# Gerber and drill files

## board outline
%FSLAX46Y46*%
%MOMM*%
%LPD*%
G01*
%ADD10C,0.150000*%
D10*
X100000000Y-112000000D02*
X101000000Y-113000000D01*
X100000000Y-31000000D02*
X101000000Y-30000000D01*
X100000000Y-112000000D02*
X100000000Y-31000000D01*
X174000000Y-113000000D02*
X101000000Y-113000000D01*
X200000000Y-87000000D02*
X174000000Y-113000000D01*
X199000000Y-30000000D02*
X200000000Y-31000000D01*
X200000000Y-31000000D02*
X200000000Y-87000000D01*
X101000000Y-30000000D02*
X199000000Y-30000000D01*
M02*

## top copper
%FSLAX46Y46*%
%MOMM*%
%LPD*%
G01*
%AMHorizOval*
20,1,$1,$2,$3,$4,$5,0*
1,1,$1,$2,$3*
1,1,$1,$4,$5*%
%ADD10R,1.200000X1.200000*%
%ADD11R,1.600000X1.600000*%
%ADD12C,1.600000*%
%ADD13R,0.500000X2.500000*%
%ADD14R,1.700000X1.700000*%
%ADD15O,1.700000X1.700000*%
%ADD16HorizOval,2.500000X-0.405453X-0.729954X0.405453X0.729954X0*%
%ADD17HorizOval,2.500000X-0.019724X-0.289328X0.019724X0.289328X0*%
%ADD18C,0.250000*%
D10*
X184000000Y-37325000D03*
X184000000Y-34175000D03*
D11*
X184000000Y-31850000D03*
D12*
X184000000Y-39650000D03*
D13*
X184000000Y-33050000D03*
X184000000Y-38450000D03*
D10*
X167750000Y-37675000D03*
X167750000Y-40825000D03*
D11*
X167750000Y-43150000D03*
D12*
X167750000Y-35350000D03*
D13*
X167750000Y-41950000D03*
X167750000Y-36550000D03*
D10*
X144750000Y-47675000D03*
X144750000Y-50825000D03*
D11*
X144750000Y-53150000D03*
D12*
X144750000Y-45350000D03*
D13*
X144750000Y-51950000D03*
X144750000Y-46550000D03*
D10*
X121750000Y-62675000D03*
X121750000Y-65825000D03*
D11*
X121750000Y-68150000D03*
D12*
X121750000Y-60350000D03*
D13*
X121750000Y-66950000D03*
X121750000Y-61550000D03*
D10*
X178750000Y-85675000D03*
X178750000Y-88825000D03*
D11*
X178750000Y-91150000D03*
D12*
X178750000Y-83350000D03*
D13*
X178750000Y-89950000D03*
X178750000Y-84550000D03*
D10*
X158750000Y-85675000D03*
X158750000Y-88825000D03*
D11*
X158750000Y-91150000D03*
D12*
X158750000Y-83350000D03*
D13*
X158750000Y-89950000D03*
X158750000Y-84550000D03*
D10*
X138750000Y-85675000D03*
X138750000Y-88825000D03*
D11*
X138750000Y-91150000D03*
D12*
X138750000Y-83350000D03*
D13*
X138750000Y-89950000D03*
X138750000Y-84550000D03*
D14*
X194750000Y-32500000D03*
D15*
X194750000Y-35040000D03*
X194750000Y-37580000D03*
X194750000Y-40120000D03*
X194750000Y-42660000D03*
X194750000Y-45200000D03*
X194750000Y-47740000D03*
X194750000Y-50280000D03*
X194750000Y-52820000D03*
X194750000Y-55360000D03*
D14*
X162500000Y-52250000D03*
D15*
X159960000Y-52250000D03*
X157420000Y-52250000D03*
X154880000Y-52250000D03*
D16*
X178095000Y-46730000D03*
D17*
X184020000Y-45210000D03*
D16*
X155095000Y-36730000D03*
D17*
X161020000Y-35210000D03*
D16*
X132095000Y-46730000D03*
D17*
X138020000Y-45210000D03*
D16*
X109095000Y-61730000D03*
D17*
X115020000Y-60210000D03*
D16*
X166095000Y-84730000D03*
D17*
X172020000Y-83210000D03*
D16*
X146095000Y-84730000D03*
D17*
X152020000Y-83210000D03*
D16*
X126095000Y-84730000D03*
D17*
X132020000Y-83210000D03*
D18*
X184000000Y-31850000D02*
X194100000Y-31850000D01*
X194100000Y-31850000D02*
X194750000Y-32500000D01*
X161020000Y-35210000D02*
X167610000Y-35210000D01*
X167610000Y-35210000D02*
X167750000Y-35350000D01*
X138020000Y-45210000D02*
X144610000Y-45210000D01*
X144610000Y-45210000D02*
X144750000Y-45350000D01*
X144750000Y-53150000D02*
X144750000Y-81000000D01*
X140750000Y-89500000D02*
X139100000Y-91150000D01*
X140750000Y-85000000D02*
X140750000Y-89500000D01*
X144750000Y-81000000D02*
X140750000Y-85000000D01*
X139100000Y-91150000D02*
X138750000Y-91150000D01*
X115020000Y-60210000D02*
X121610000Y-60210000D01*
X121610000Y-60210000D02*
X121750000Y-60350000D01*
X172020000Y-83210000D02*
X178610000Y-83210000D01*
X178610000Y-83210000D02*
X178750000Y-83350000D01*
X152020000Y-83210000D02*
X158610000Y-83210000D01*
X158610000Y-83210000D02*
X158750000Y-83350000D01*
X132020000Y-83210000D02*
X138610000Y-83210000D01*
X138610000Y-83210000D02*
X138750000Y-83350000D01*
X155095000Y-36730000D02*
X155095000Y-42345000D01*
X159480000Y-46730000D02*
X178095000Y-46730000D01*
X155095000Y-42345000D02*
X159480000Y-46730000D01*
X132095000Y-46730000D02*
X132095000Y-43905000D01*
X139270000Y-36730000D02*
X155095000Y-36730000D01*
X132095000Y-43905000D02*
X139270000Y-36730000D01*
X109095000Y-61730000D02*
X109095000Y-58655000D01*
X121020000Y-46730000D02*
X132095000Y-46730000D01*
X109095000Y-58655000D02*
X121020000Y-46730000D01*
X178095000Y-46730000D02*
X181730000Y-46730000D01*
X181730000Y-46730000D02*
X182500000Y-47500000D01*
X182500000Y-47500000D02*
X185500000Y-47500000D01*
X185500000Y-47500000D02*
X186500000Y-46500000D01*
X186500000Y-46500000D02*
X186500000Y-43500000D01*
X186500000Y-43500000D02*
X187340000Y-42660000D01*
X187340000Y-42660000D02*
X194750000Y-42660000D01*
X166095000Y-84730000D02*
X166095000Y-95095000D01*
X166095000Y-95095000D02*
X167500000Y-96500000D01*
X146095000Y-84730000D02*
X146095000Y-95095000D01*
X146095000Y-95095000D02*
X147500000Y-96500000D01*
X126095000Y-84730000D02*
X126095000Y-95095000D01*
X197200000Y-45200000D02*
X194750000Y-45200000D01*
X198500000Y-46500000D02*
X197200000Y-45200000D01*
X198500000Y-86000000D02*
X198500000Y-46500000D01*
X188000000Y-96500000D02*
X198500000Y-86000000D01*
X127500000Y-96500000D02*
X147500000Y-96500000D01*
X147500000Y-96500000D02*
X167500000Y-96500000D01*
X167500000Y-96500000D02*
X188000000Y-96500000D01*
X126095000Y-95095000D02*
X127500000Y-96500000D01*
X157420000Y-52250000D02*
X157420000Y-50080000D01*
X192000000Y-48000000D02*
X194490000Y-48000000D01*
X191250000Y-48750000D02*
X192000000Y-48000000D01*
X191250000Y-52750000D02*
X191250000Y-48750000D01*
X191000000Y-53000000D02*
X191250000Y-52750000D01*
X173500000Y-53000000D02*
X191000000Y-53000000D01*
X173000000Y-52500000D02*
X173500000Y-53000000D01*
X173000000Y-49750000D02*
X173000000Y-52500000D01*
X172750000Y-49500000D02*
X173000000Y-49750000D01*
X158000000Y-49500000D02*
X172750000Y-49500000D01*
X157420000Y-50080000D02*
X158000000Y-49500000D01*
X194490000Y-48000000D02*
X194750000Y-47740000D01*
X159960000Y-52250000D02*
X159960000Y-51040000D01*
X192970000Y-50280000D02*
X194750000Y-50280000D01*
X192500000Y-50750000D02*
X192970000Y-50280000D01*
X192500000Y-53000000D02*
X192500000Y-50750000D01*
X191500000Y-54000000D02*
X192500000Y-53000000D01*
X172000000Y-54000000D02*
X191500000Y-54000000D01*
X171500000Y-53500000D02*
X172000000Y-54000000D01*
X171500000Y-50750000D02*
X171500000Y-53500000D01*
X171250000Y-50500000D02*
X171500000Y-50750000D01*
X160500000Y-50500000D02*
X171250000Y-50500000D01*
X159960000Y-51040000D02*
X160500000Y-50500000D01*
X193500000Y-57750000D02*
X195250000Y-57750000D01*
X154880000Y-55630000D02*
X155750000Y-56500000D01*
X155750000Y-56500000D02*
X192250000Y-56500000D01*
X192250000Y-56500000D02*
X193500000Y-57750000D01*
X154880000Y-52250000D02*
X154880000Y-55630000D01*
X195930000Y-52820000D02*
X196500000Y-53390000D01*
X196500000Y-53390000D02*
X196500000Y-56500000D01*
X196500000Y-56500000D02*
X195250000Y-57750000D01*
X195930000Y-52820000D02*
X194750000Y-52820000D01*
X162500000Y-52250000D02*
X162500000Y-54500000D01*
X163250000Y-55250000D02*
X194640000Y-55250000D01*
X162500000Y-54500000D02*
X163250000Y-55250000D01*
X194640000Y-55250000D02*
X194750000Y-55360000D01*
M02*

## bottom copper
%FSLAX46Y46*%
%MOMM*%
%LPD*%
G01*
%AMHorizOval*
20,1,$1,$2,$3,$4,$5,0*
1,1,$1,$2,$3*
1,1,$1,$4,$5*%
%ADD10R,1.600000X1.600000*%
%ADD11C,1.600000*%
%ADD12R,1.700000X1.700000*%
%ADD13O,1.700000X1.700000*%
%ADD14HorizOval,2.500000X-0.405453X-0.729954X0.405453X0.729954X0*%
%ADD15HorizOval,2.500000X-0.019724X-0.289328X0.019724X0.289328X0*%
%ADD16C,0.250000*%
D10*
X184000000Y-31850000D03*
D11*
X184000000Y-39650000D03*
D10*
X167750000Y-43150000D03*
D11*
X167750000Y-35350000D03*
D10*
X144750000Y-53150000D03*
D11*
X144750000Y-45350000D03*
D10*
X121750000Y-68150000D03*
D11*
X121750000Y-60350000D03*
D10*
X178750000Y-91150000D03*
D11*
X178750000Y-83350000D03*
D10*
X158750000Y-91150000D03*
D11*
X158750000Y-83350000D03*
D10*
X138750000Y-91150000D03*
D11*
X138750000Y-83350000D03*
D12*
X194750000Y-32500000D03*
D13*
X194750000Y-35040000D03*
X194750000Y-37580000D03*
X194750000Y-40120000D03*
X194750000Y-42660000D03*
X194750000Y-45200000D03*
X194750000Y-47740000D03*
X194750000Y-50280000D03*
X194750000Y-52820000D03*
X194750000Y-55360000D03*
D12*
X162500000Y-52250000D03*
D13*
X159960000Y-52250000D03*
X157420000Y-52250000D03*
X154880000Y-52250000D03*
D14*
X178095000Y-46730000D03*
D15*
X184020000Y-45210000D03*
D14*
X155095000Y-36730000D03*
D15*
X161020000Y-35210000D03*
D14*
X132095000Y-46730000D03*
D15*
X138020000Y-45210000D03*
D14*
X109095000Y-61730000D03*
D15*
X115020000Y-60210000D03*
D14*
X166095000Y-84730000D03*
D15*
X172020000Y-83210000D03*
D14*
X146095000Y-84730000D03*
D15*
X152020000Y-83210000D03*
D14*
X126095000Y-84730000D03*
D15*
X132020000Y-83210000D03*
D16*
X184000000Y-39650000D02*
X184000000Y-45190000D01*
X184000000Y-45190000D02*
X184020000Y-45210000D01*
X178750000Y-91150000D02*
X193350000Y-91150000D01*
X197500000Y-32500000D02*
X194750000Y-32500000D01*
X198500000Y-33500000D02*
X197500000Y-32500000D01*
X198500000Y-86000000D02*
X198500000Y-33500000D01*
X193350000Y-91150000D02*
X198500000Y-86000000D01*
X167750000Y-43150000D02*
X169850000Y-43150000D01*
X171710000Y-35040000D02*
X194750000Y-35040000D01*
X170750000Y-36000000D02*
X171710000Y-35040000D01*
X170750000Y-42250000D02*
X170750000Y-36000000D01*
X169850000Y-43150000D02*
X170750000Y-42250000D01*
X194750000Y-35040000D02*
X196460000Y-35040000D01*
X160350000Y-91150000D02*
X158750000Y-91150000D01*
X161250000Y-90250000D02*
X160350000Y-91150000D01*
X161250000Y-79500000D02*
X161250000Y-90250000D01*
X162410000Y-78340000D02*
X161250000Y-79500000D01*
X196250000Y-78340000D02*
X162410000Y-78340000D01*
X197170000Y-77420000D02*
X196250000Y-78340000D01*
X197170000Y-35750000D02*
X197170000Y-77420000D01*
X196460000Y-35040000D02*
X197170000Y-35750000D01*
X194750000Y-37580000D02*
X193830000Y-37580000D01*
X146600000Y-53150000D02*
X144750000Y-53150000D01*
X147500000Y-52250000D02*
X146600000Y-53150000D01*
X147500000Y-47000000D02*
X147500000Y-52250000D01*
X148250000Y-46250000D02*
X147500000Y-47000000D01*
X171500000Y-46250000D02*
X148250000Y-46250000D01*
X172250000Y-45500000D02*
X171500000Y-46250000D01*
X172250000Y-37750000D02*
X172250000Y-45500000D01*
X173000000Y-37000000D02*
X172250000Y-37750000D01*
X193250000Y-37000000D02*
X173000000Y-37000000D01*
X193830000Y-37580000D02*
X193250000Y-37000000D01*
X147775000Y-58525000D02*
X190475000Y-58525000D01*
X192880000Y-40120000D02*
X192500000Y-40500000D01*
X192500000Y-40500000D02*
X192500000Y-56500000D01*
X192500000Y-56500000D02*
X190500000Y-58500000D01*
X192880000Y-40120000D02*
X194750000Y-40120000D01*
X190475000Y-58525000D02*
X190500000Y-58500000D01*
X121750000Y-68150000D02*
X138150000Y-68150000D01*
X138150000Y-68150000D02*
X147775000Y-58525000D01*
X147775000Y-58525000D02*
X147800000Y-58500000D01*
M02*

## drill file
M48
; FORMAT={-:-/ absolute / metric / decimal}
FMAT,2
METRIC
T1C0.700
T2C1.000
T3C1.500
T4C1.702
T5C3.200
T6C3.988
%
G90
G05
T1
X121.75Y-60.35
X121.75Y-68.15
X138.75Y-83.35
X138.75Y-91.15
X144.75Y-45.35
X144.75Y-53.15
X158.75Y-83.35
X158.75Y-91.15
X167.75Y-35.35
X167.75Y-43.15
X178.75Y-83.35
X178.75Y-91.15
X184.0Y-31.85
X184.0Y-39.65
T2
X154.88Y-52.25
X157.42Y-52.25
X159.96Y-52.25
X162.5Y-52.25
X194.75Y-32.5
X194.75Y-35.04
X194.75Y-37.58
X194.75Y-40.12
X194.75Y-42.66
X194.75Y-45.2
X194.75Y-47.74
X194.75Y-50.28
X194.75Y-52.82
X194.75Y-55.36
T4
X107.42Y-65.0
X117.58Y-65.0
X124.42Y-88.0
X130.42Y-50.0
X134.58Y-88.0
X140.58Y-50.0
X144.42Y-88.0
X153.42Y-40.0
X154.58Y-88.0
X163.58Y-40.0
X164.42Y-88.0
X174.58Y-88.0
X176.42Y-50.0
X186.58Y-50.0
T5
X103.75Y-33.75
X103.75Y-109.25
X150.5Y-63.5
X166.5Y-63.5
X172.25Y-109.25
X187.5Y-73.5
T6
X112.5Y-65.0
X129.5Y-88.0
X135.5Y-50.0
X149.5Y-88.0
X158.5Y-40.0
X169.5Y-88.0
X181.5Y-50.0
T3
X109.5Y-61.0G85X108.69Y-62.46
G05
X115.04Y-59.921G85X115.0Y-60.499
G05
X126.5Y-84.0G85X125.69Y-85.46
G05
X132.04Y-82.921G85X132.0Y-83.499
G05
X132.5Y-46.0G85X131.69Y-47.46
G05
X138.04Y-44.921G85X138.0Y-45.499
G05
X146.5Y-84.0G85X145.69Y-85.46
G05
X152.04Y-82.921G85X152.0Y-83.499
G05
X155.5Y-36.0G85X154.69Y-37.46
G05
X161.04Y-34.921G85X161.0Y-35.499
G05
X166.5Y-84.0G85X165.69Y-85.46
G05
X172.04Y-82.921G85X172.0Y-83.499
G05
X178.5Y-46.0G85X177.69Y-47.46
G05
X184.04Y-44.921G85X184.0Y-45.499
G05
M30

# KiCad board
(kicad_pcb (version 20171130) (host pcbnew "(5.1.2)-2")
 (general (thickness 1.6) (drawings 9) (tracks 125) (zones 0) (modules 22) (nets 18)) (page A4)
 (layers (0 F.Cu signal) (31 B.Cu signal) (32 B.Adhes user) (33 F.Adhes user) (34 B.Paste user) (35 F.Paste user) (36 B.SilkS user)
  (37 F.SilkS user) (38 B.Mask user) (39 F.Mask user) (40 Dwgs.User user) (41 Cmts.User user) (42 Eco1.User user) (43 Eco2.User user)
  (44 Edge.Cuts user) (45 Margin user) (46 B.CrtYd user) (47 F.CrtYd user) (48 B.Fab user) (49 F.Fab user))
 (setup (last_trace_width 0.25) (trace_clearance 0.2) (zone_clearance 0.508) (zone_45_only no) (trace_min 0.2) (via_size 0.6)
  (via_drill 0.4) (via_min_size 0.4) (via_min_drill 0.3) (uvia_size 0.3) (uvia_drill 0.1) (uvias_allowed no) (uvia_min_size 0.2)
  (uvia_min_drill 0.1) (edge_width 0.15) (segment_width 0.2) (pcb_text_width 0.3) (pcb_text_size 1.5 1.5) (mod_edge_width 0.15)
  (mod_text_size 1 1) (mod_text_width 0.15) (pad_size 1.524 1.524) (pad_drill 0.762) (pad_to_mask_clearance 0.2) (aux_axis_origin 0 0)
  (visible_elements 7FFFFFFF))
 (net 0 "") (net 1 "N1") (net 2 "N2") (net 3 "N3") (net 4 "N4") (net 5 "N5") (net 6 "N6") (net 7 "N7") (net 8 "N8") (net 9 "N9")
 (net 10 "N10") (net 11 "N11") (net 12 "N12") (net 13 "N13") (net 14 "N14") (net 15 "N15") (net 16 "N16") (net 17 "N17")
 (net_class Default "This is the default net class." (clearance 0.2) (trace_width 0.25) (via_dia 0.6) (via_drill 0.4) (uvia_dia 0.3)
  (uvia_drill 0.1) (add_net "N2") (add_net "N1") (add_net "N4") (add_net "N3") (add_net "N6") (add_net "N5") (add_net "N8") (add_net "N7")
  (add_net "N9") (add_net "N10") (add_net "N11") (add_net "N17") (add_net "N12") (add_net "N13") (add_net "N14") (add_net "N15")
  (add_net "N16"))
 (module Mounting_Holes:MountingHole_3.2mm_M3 (layer F.Cu) (at 187.5 73.5)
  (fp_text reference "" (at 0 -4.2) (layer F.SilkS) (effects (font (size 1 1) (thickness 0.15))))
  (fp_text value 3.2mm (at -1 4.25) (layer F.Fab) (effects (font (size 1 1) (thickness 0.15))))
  (pad 1 np_thru_hole circle (at 0 0) (size 3.2 3.2) (drill 3.2) (layers *.Cu *.Mask)))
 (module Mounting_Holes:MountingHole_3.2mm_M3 (layer F.Cu) (at 172.25 109.25)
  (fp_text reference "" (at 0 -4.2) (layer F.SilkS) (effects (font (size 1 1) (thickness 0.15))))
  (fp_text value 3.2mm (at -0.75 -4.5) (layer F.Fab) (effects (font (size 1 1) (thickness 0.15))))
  (pad 1 np_thru_hole circle (at 0 0) (size 3.2 3.2) (drill 3.2) (layers *.Cu *.Mask)))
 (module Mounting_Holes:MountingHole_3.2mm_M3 (layer F.Cu) (at 103.75 109.25)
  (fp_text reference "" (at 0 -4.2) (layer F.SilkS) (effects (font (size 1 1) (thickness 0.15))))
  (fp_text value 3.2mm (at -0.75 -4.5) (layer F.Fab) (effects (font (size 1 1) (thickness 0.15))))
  (pad 1 np_thru_hole circle (at 0 0) (size 3.2 3.2) (drill 3.2) (layers *.Cu *.Mask)))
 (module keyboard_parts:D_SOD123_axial (layer F.Cu) (at 184 35.75 270)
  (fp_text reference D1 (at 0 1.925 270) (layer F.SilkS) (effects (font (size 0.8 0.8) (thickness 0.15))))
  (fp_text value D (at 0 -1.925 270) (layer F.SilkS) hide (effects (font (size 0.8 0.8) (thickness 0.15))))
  (pad 2 smd rect (at 1.575 0 270) (size 1.2 1.2) (layers F.Cu F.Paste F.Mask) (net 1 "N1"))
  (pad 1 smd rect (at -1.575 0 270) (size 1.2 1.2) (layers F.Cu F.Paste F.Mask) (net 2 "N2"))
  (pad 1 thru_hole rect (at -3.9 0 270) (size 1.6 1.6) (drill 0.7) (layers *.Cu *.Mask F.SilkS) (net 2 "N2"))
  (pad 2 thru_hole circle (at 3.9 0 270) (size 1.6 1.6) (drill 0.7) (layers *.Cu *.Mask F.SilkS) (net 1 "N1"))
  (pad 1 smd rect (at -2.7 0 270) (size 2.5 0.5) (layers F.Cu) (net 2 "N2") (solder_mask_margin -999))
  (pad 2 smd rect (at 2.7 0 270) (size 2.5 0.5) (layers F.Cu) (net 1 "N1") (solder_mask_margin -999)))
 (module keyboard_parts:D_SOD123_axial (layer F.Cu) (at 167.75 39.25 90)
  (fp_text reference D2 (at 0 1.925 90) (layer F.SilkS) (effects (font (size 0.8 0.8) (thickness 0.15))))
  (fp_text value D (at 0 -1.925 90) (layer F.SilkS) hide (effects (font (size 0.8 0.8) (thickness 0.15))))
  (pad 2 smd rect (at 1.575 0 90) (size 1.2 1.2) (layers F.Cu F.Paste F.Mask) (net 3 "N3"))
  (pad 1 smd rect (at -1.575 0 90) (size 1.2 1.2) (layers F.Cu F.Paste F.Mask) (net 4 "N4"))
  (pad 1 thru_hole rect (at -3.9 0 90) (size 1.6 1.6) (drill 0.7) (layers *.Cu *.Mask F.SilkS) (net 4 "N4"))
  (pad 2 thru_hole circle (at 3.9 0 90) (size 1.6 1.6) (drill 0.7) (layers *.Cu *.Mask F.SilkS) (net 3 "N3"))
  (pad 1 smd rect (at -2.7 0 90) (size 2.5 0.5) (layers F.Cu) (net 4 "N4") (solder_mask_margin -999))
  (pad 2 smd rect (at 2.7 0 90) (size 2.5 0.5) (layers F.Cu) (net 3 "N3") (solder_mask_margin -999)))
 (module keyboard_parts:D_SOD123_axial (layer F.Cu) (at 144.75 49.25 90)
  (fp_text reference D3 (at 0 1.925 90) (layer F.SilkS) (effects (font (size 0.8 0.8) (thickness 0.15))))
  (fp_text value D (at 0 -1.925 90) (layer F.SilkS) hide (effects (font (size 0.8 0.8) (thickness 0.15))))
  (pad 2 smd rect (at 1.575 0 90) (size 1.2 1.2) (layers F.Cu F.Paste F.Mask) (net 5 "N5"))
  (pad 1 smd rect (at -1.575 0 90) (size 1.2 1.2) (layers F.Cu F.Paste F.Mask) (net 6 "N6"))
  (pad 1 thru_hole rect (at -3.9 0 90) (size 1.6 1.6) (drill 0.7) (layers *.Cu *.Mask F.SilkS) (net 6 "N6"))
  (pad 2 thru_hole circle (at 3.9 0 90) (size 1.6 1.6) (drill 0.7) (layers *.Cu *.Mask F.SilkS) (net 5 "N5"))
  (pad 1 smd rect (at -2.7 0 90) (size 2.5 0.5) (layers F.Cu) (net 6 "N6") (solder_mask_margin -999))
  (pad 2 smd rect (at 2.7 0 90) (size 2.5 0.5) (layers F.Cu) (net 5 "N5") (solder_mask_margin -999)))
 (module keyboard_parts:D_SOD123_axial (layer F.Cu) (at 121.75 64.25 90)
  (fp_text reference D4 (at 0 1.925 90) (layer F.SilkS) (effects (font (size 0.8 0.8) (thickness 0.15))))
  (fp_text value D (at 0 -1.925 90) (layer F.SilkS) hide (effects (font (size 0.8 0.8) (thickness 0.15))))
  (pad 2 smd rect (at 1.575 0 90) (size 1.2 1.2) (layers F.Cu F.Paste F.Mask) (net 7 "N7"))
  (pad 1 smd rect (at -1.575 0 90) (size 1.2 1.2) (layers F.Cu F.Paste F.Mask) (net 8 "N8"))
  (pad 1 thru_hole rect (at -3.9 0 90) (size 1.6 1.6) (drill 0.7) (layers *.Cu *.Mask F.SilkS) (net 8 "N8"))
  (pad 2 thru_hole circle (at 3.9 0 90) (size 1.6 1.6) (drill 0.7) (layers *.Cu *.Mask F.SilkS) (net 7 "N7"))
  (pad 1 smd rect (at -2.7 0 90) (size 2.5 0.5) (layers F.Cu) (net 8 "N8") (solder_mask_margin -999))
  (pad 2 smd rect (at 2.7 0 90) (size 2.5 0.5) (layers F.Cu) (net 7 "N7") (solder_mask_margin -999)))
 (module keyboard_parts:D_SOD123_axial (layer F.Cu) (at 178.75 87.25 90)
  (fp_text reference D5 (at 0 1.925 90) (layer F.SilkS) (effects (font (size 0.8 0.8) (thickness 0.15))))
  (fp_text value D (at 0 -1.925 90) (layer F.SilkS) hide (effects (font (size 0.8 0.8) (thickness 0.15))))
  (pad 2 smd rect (at 1.575 0 90) (size 1.2 1.2) (layers F.Cu F.Paste F.Mask) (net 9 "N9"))
  (pad 1 smd rect (at -1.575 0 90) (size 1.2 1.2) (layers F.Cu F.Paste F.Mask) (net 2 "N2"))
  (pad 1 thru_hole rect (at -3.9 0 90) (size 1.6 1.6) (drill 0.7) (layers *.Cu *.Mask F.SilkS) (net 2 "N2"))
  (pad 2 thru_hole circle (at 3.9 0 90) (size 1.6 1.6) (drill 0.7) (layers *.Cu *.Mask F.SilkS) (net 9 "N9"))
  (pad 1 smd rect (at -2.7 0 90) (size 2.5 0.5) (layers F.Cu) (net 2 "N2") (solder_mask_margin -999))
  (pad 2 smd rect (at 2.7 0 90) (size 2.5 0.5) (layers F.Cu) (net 9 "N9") (solder_mask_margin -999)))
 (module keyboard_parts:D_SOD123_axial (layer F.Cu) (at 158.75 87.25 90)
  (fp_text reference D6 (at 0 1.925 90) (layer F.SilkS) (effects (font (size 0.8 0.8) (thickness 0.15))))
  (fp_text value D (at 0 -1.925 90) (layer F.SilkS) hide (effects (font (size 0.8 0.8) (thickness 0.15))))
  (pad 2 smd rect (at 1.575 0 90) (size 1.2 1.2) (layers F.Cu F.Paste F.Mask) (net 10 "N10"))
  (pad 1 smd rect (at -1.575 0 90) (size 1.2 1.2) (layers F.Cu F.Paste F.Mask) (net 4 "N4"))
  (pad 1 thru_hole rect (at -3.9 0 90) (size 1.6 1.6) (drill 0.7) (layers *.Cu *.Mask F.SilkS) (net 4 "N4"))
  (pad 2 thru_hole circle (at 3.9 0 90) (size 1.6 1.6) (drill 0.7) (layers *.Cu *.Mask F.SilkS) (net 10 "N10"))
  (pad 1 smd rect (at -2.7 0 90) (size 2.5 0.5) (layers F.Cu) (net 4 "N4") (solder_mask_margin -999))
  (pad 2 smd rect (at 2.7 0 90) (size 2.5 0.5) (layers F.Cu) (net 10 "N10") (solder_mask_margin -999)))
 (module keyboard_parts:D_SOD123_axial (layer F.Cu) (at 138.75 87.25 90)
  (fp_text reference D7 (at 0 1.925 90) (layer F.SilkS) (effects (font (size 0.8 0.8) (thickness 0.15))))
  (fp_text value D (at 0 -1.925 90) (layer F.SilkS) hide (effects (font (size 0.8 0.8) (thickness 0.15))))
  (pad 2 smd rect (at 1.575 0 90) (size 1.2 1.2) (layers F.Cu F.Paste F.Mask) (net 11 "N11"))
  (pad 1 smd rect (at -1.575 0 90) (size 1.2 1.2) (layers F.Cu F.Paste F.Mask) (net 6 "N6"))
  (pad 1 thru_hole rect (at -3.9 0 90) (size 1.6 1.6) (drill 0.7) (layers *.Cu *.Mask F.SilkS) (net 6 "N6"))
  (pad 2 thru_hole circle (at 3.9 0 90) (size 1.6 1.6) (drill 0.7) (layers *.Cu *.Mask F.SilkS) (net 11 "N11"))
  (pad 1 smd rect (at -2.7 0 90) (size 2.5 0.5) (layers F.Cu) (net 6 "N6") (solder_mask_margin -999))
  (pad 2 smd rect (at 2.7 0 90) (size 2.5 0.5) (layers F.Cu) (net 11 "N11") (solder_mask_margin -999)))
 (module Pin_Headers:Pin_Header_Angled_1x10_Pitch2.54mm (layer F.Cu) (at 194.75 32.5)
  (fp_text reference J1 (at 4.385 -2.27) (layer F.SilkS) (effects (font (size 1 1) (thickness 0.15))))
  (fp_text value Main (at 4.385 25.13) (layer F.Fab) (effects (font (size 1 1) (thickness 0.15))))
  (pad 1 thru_hole rect (at 0 0) (size 1.7 1.7) (drill 1) (layers *.Cu *.Mask) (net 2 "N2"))
  (pad 2 thru_hole oval (at 0 2.54) (size 1.7 1.7) (drill 1) (layers *.Cu *.Mask) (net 4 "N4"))
  (pad 3 thru_hole oval (at 0 5.08) (size 1.7 1.7) (drill 1) (layers *.Cu *.Mask) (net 6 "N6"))
  (pad 4 thru_hole oval (at 0 7.62) (size 1.7 1.7) (drill 1) (layers *.Cu *.Mask) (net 8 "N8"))
  (pad 5 thru_hole oval (at 0 10.16) (size 1.7 1.7) (drill 1) (layers *.Cu *.Mask) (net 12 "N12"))
  (pad 6 thru_hole oval (at 0 12.7) (size 1.7 1.7) (drill 1) (layers *.Cu *.Mask) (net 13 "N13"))
  (pad 7 thru_hole oval (at 0 15.24) (size 1.7 1.7) (drill 1) (layers *.Cu *.Mask) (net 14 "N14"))
  (pad 8 thru_hole oval (at 0 17.78) (size 1.7 1.7) (drill 1) (layers *.Cu *.Mask) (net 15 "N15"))
  (pad 9 thru_hole oval (at 0 20.32) (size 1.7 1.7) (drill 1) (layers *.Cu *.Mask) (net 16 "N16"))
  (pad 10 thru_hole oval (at 0 22.86) (size 1.7 1.7) (drill 1) (layers *.Cu *.Mask) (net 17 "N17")))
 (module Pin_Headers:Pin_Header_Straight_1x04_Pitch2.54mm (layer F.Cu) (at 162.5 52.25 270)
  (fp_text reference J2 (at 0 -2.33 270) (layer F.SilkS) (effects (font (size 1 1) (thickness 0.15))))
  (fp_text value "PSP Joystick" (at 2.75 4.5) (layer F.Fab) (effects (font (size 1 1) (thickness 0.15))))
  (pad 1 thru_hole rect (at 0 0 270) (size 1.7 1.7) (drill 1) (layers *.Cu *.Mask) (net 17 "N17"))
  (pad 2 thru_hole oval (at 0 2.54 270) (size 1.7 1.7) (drill 1) (layers *.Cu *.Mask) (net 15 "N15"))
  (pad 3 thru_hole oval (at 0 5.08 270) (size 1.7 1.7) (drill 1) (layers *.Cu *.Mask) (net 14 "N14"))
  (pad 4 thru_hole oval (at 0 7.62 270) (size 1.7 1.7) (drill 1) (layers *.Cu *.Mask) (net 16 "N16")))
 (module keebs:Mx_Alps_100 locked (layer F.Cu) (at 181.5 50)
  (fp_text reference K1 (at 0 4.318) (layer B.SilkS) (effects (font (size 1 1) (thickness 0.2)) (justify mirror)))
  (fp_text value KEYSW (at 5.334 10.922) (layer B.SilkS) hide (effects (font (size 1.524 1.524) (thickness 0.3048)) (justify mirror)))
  (pad HOLE np_thru_hole circle (at 0 0) (size 3.9878 3.9878) (drill 3.9878) (layers *.Cu))
  (pad HOLE np_thru_hole circle (at -5.08 0) (size 1.7018 1.7018) (drill 1.7018) (layers *.Cu))
  (pad HOLE np_thru_hole circle (at 5.08 0) (size 1.7018 1.7018) (drill 1.7018) (layers *.Cu))
  (pad 1 thru_hole oval (at -3.405 -3.27 330.95) (size 2.5 4.17) (drill oval 1.5 3.17) (layers *.Cu *.Mask F.SilkS) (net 12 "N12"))
  (pad 2 thru_hole oval (at 2.52 -4.79 356.1) (size 2.5 3.08) (drill oval 1.5 2.08) (layers *.Cu *.Mask F.SilkS) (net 1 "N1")))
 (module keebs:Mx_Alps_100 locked (layer F.Cu) (at 158.5 40)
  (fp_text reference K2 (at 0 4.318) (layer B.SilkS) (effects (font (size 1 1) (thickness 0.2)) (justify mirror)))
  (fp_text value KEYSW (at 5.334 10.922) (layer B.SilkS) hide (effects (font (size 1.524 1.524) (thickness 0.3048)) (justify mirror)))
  (pad HOLE np_thru_hole circle (at 0 0) (size 3.9878 3.9878) (drill 3.9878) (layers *.Cu))
  (pad HOLE np_thru_hole circle (at -5.08 0) (size 1.7018 1.7018) (drill 1.7018) (layers *.Cu))
  (pad HOLE np_thru_hole circle (at 5.08 0) (size 1.7018 1.7018) (drill 1.7018) (layers *.Cu))
  (pad 1 thru_hole oval (at -3.405 -3.27 330.95) (size 2.5 4.17) (drill oval 1.5 3.17) (layers *.Cu *.Mask F.SilkS) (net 12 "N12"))
  (pad 2 thru_hole oval (at 2.52 -4.79 356.1) (size 2.5 3.08) (drill oval 1.5 2.08) (layers *.Cu *.Mask F.SilkS) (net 3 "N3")))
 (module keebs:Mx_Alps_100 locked (layer F.Cu) (at 135.5 50)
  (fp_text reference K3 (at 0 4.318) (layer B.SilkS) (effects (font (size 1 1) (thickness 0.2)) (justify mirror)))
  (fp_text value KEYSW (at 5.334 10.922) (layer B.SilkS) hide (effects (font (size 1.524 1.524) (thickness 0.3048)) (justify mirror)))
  (pad HOLE np_thru_hole circle (at 0 0) (size 3.9878 3.9878) (drill 3.9878) (layers *.Cu))
  (pad HOLE np_thru_hole circle (at -5.08 0) (size 1.7018 1.7018) (drill 1.7018) (layers *.Cu))
  (pad HOLE np_thru_hole circle (at 5.08 0) (size 1.7018 1.7018) (drill 1.7018) (layers *.Cu))
  (pad 1 thru_hole oval (at -3.405 -3.27 330.95) (size 2.5 4.17) (drill oval 1.5 3.17) (layers *.Cu *.Mask F.SilkS) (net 12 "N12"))
  (pad 2 thru_hole oval (at 2.52 -4.79 356.1) (size 2.5 3.08) (drill oval 1.5 2.08) (layers *.Cu *.Mask F.SilkS) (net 5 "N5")))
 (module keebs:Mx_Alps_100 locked (layer F.Cu) (at 112.5 65)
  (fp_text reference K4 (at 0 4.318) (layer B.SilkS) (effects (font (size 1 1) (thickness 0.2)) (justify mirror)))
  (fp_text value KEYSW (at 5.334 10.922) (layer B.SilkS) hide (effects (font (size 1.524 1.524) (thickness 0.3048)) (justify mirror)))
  (pad HOLE np_thru_hole circle (at 0 0) (size 3.9878 3.9878) (drill 3.9878) (layers *.Cu))
  (pad HOLE np_thru_hole circle (at -5.08 0) (size 1.7018 1.7018) (drill 1.7018) (layers *.Cu))
  (pad HOLE np_thru_hole circle (at 5.08 0) (size 1.7018 1.7018) (drill 1.7018) (layers *.Cu))
  (pad 1 thru_hole oval (at -3.405 -3.27 330.95) (size 2.5 4.17) (drill oval 1.5 3.17) (layers *.Cu *.Mask F.SilkS) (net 12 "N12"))
  (pad 2 thru_hole oval (at 2.52 -4.79 356.1) (size 2.5 3.08) (drill oval 1.5 2.08) (layers *.Cu *.Mask F.SilkS) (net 7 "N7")))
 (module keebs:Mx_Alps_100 (layer F.Cu) (at 169.5 88)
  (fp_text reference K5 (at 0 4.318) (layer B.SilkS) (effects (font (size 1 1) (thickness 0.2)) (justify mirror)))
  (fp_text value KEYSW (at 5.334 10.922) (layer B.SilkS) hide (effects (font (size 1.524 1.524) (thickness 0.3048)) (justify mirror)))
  (pad HOLE np_thru_hole circle (at 0 0) (size 3.9878 3.9878) (drill 3.9878) (layers *.Cu))
  (pad HOLE np_thru_hole circle (at -5.08 0) (size 1.7018 1.7018) (drill 1.7018) (layers *.Cu))
  (pad HOLE np_thru_hole circle (at 5.08 0) (size 1.7018 1.7018) (drill 1.7018) (layers *.Cu))
  (pad 1 thru_hole oval (at -3.405 -3.27 330.95) (size 2.5 4.17) (drill oval 1.5 3.17) (layers *.Cu *.Mask F.SilkS) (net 13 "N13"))
  (pad 2 thru_hole oval (at 2.52 -4.79 356.1) (size 2.5 3.08) (drill oval 1.5 2.08) (layers *.Cu *.Mask F.SilkS) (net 9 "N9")))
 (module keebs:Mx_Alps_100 (layer F.Cu) (at 149.5 88)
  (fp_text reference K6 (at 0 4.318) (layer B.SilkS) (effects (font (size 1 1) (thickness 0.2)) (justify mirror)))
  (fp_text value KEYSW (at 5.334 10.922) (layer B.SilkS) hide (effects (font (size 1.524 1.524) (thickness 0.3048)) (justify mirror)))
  (pad HOLE np_thru_hole circle (at 0 0) (size 3.9878 3.9878) (drill 3.9878) (layers *.Cu))
  (pad HOLE np_thru_hole circle (at -5.08 0) (size 1.7018 1.7018) (drill 1.7018) (layers *.Cu))
  (pad HOLE np_thru_hole circle (at 5.08 0) (size 1.7018 1.7018) (drill 1.7018) (layers *.Cu))
  (pad 1 thru_hole oval (at -3.405 -3.27 330.95) (size 2.5 4.17) (drill oval 1.5 3.17) (layers *.Cu *.Mask F.SilkS) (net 13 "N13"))
  (pad 2 thru_hole oval (at 2.52 -4.79 356.1) (size 2.5 3.08) (drill oval 1.5 2.08) (layers *.Cu *.Mask F.SilkS) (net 10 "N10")))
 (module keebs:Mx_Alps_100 (layer F.Cu) (at 129.5 88)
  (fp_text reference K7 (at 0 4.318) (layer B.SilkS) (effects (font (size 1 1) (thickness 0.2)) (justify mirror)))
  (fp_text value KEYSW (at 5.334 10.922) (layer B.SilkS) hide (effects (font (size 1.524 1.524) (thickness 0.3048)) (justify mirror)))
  (pad HOLE np_thru_hole circle (at 0 0) (size 3.9878 3.9878) (drill 3.9878) (layers *.Cu))
  (pad HOLE np_thru_hole circle (at -5.08 0) (size 1.7018 1.7018) (drill 1.7018) (layers *.Cu))
  (pad HOLE np_thru_hole circle (at 5.08 0) (size 1.7018 1.7018) (drill 1.7018) (layers *.Cu))
  (pad 1 thru_hole oval (at -3.405 -3.27 330.95) (size 2.5 4.17) (drill oval 1.5 3.17) (layers *.Cu *.Mask F.SilkS) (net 13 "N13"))
  (pad 2 thru_hole oval (at 2.52 -4.79 356.1) (size 2.5 3.08) (drill oval 1.5 2.08) (layers *.Cu *.Mask F.SilkS) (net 11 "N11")))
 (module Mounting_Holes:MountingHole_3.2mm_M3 (layer F.Cu) (at 166.5 63.5)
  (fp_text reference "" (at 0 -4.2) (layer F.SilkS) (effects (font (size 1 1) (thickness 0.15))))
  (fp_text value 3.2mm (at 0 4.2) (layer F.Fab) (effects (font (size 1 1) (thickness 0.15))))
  (pad 1 np_thru_hole circle (at 0 0) (size 3.2 3.2) (drill 3.2) (layers *.Cu *.Mask)))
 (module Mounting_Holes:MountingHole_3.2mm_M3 (layer F.Cu) (at 150.5 63.5)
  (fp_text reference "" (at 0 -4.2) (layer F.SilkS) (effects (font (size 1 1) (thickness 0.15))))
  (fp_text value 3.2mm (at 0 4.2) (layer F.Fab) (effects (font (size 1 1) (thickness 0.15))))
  (pad 1 np_thru_hole circle (at 0 0) (size 3.2 3.2) (drill 3.2) (layers *.Cu *.Mask)))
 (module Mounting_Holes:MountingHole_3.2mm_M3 (layer F.Cu) (at 103.75 33.75)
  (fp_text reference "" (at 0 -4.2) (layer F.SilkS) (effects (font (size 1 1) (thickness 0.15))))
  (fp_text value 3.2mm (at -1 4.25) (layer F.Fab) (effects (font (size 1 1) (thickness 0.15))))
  (pad 1 np_thru_hole circle (at 0 0) (size 3.2 3.2) (drill 3.2) (layers *.Cu *.Mask)))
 (gr_line (start 100 112) (end 101 113) (angle 90) (layer Edge.Cuts) (width 0.15))
 (gr_line (start 100 31) (end 101 30) (angle 90) (layer Edge.Cuts) (width 0.15))
 (gr_line (start 100 112) (end 100 31) (angle 90) (layer Edge.Cuts) (width 0.15))
 (gr_line (start 174 113) (end 101 113) (angle 90) (layer Edge.Cuts) (width 0.15))
 (gr_line (start 200 87) (end 174 113) (angle 90) (layer Edge.Cuts) (width 0.15))
 (gr_line (start 199 30) (end 200 31) (angle 90) (layer Edge.Cuts) (width 0.15))
 (gr_line (start 200 31) (end 200 87) (angle 90) (layer Edge.Cuts) (width 0.15))
 (gr_line (start 101 30) (end 199 30) (angle 90) (layer Edge.Cuts) (width 0.15))
 (segment (start 184 39.65) (end 184 45.19) (width 0.25) (layer B.Cu) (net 1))
 (segment (start 184 45.19) (end 184.02 45.21) (width 0.25) (layer B.Cu) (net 1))
 (segment (start 184 31.85) (end 194.1 31.85) (width 0.25) (layer F.Cu) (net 2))
 (segment (start 194.1 31.85) (end 194.75 32.5) (width 0.25) (layer F.Cu) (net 2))
 (segment (start 178.75 91.15) (end 193.35 91.15) (width 0.25) (layer B.Cu) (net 2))
 (segment (start 197.5 32.5) (end 194.75 32.5) (width 0.25) (layer B.Cu) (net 2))
 (segment (start 198.5 33.5) (end 197.5 32.5) (width 0.25) (layer B.Cu) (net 2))
 (segment (start 198.5 86) (end 198.5 33.5) (width 0.25) (layer B.Cu) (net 2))
 (segment (start 193.35 91.15) (end 198.5 86) (width 0.25) (layer B.Cu) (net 2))
 (segment (start 161.02 35.21) (end 167.61 35.21) (width 0.25) (layer F.Cu) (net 3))
 (segment (start 167.61 35.21) (end 167.75 35.35) (width 0.25) (layer F.Cu) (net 3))
 (segment (start 167.75 43.15) (end 169.85 43.15) (width 0.25) (layer B.Cu) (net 4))
 (segment (start 171.71 35.04) (end 194.75 35.04) (width 0.25) (layer B.Cu) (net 4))
 (segment (start 170.75 36) (end 171.71 35.04) (width 0.25) (layer B.Cu) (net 4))
 (segment (start 170.75 42.25) (end 170.75 36) (width 0.25) (layer B.Cu) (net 4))
 (segment (start 169.85 43.15) (end 170.75 42.25) (width 0.25) (layer B.Cu) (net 4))
 (segment (start 194.75 35.04) (end 196.46 35.04) (width 0.25) (layer B.Cu) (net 4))
 (segment (start 160.35 91.15) (end 158.75 91.15) (width 0.25) (layer B.Cu) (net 4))
 (segment (start 161.25 90.25) (end 160.35 91.15) (width 0.25) (layer B.Cu) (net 4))
 (segment (start 161.25 79.5) (end 161.25 90.25) (width 0.25) (layer B.Cu) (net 4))
 (segment (start 162.41 78.34) (end 161.25 79.5) (width 0.25) (layer B.Cu) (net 4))
 (segment (start 196.25 78.34) (end 162.41 78.34) (width 0.25) (layer B.Cu) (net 4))
 (segment (start 197.17 77.42) (end 196.25 78.34) (width 0.25) (layer B.Cu) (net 4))
 (segment (start 197.17 35.75) (end 197.17 77.42) (width 0.25) (layer B.Cu) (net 4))
 (segment (start 196.46 35.04) (end 197.17 35.75) (width 0.25) (layer B.Cu) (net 4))
 (segment (start 138.02 45.21) (end 144.61 45.21) (width 0.25) (layer F.Cu) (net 5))
 (segment (start 144.61 45.21) (end 144.75 45.35) (width 0.25) (layer F.Cu) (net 5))
 (segment (start 144.75 53.15) (end 144.75 81) (width 0.25) (layer F.Cu) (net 6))
 (segment (start 140.75 89.5) (end 139.1 91.15) (width 0.25) (layer F.Cu) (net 6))
 (segment (start 140.75 85) (end 140.75 89.5) (width 0.25) (layer F.Cu) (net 6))
 (segment (start 144.75 81) (end 140.75 85) (width 0.25) (layer F.Cu) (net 6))
 (segment (start 139.1 91.15) (end 138.75 91.15) (width 0.25) (layer F.Cu) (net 6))
 (segment (start 194.75 37.58) (end 193.83 37.58) (width 0.25) (layer B.Cu) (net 6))
 (segment (start 146.6 53.15) (end 144.75 53.15) (width 0.25) (layer B.Cu) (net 6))
 (segment (start 147.5 52.25) (end 146.6 53.15) (width 0.25) (layer B.Cu) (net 6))
 (segment (start 147.5 47) (end 147.5 52.25) (width 0.25) (layer B.Cu) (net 6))
 (segment (start 148.25 46.25) (end 147.5 47) (width 0.25) (layer B.Cu) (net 6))
 (segment (start 171.5 46.25) (end 148.25 46.25) (width 0.25) (layer B.Cu) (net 6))
 (segment (start 172.25 45.5) (end 171.5 46.25) (width 0.25) (layer B.Cu) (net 6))
 (segment (start 172.25 37.75) (end 172.25 45.5) (width 0.25) (layer B.Cu) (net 6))
 (segment (start 173 37) (end 172.25 37.75) (width 0.25) (layer B.Cu) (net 6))
 (segment (start 193.25 37) (end 173 37) (width 0.25) (layer B.Cu) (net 6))
 (segment (start 193.83 37.58) (end 193.25 37) (width 0.25) (layer B.Cu) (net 6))
 (segment (start 115.02 60.21) (end 121.61 60.21) (width 0.25) (layer F.Cu) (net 7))
 (segment (start 121.61 60.21) (end 121.75 60.35) (width 0.25) (layer F.Cu) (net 7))
 (segment (start 147.775 58.525) (end 190.475 58.525) (width 0.25) (layer B.Cu) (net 8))
 (segment (start 192.88 40.12) (end 192.5 40.5) (width 0.25) (layer B.Cu) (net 8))
 (segment (start 192.5 40.5) (end 192.5 56.5) (width 0.25) (layer B.Cu) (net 8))
 (segment (start 192.5 56.5) (end 190.5 58.5) (width 0.25) (layer B.Cu) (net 8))
 (segment (start 192.88 40.12) (end 194.75 40.12) (width 0.25) (layer B.Cu) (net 8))
 (segment (start 190.475 58.525) (end 190.5 58.5) (width 0.25) (layer B.Cu) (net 8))
 (segment (start 121.75 68.15) (end 138.15 68.15) (width 0.25) (layer B.Cu) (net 8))
 (segment (start 138.15 68.15) (end 147.775 58.525) (width 0.25) (layer B.Cu) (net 8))
 (segment (start 147.775 58.525) (end 147.8 58.5) (width 0.25) (layer B.Cu) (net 8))
 (segment (start 172.02 83.21) (end 178.61 83.21) (width 0.25) (layer F.Cu) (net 9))
 (segment (start 178.61 83.21) (end 178.75 83.35) (width 0.25) (layer F.Cu) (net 9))
 (segment (start 152.02 83.21) (end 158.61 83.21) (width 0.25) (layer F.Cu) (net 10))
 (segment (start 158.61 83.21) (end 158.75 83.35) (width 0.25) (layer F.Cu) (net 10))
 (segment (start 132.02 83.21) (end 138.61 83.21) (width 0.25) (layer F.Cu) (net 11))
 (segment (start 138.61 83.21) (end 138.75 83.35) (width 0.25) (layer F.Cu) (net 11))
 (segment (start 155.095 36.73) (end 155.095 42.345) (width 0.25) (layer F.Cu) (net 12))
 (segment (start 159.48 46.73) (end 178.095 46.73) (width 0.25) (layer F.Cu) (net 12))
 (segment (start 155.095 42.345) (end 159.48 46.73) (width 0.25) (layer F.Cu) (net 12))
 (segment (start 132.095 46.73) (end 132.095 43.905) (width 0.25) (layer F.Cu) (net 12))
 (segment (start 139.27 36.73) (end 155.095 36.73) (width 0.25) (layer F.Cu) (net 12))
 (segment (start 132.095 43.905) (end 139.27 36.73) (width 0.25) (layer F.Cu) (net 12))
 (segment (start 109.095 61.73) (end 109.095 58.655) (width 0.25) (layer F.Cu) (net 12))
 (segment (start 121.02 46.73) (end 132.095 46.73) (width 0.25) (layer F.Cu) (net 12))
 (segment (start 109.095 58.655) (end 121.02 46.73) (width 0.25) (layer F.Cu) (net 12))
 (segment (start 178.095 46.73) (end 181.73 46.73) (width 0.25) (layer F.Cu) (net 12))
 (segment (start 181.73 46.73) (end 182.5 47.5) (width 0.25) (layer F.Cu) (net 12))
 (segment (start 182.5 47.5) (end 185.5 47.5) (width 0.25) (layer F.Cu) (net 12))
 (segment (start 185.5 47.5) (end 186.5 46.5) (width 0.25) (layer F.Cu) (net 12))
 (segment (start 186.5 46.5) (end 186.5 43.5) (width 0.25) (layer F.Cu) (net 12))
 (segment (start 186.5 43.5) (end 187.34 42.66) (width 0.25) (layer F.Cu) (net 12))
 (segment (start 187.34 42.66) (end 194.75 42.66) (width 0.25) (layer F.Cu) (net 12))
 (segment (start 166.095 84.73) (end 166.095 95.095) (width 0.25) (layer F.Cu) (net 13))
 (segment (start 166.095 95.095) (end 167.5 96.5) (width 0.25) (layer F.Cu) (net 13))
 (segment (start 146.095 84.73) (end 146.095 95.095) (width 0.25) (layer F.Cu) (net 13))
 (segment (start 146.095 95.095) (end 147.5 96.5) (width 0.25) (layer F.Cu) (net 13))
 (segment (start 126.095 84.73) (end 126.095 95.095) (width 0.25) (layer F.Cu) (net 13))
 (segment (start 197.2 45.2) (end 194.75 45.2) (width 0.25) (layer F.Cu) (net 13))
 (segment (start 198.5 46.5) (end 197.2 45.2) (width 0.25) (layer F.Cu) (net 13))
 (segment (start 198.5 86) (end 198.5 46.5) (width 0.25) (layer F.Cu) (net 13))
 (segment (start 188 96.5) (end 198.5 86) (width 0.25) (layer F.Cu) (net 13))
 (segment (start 127.5 96.5) (end 147.5 96.5) (width 0.25) (layer F.Cu) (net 13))
 (segment (start 147.5 96.5) (end 167.5 96.5) (width 0.25) (layer F.Cu) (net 13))
 (segment (start 167.5 96.5) (end 188 96.5) (width 0.25) (layer F.Cu) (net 13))
 (segment (start 126.095 95.095) (end 127.5 96.5) (width 0.25) (layer F.Cu) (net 13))
 (segment (start 157.42 52.25) (end 157.42 50.08) (width 0.25) (layer F.Cu) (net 14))
 (segment (start 192 48) (end 194.49 48) (width 0.25) (layer F.Cu) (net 14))
 (segment (start 191.25 48.75) (end 192 48) (width 0.25) (layer F.Cu) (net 14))
 (segment (start 191.25 52.75) (end 191.25 48.75) (width 0.25) (layer F.Cu) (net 14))
 (segment (start 191 53) (end 191.25 52.75) (width 0.25) (layer F.Cu) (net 14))
 (segment (start 173.5 53) (end 191 53) (width 0.25) (layer F.Cu) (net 14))
 (segment (start 173 52.5) (end 173.5 53) (width 0.25) (layer F.Cu) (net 14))
 (segment (start 173 49.75) (end 173 52.5) (width 0.25) (layer F.Cu) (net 14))
 (segment (start 172.75 49.5) (end 173 49.75) (width 0.25) (layer F.Cu) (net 14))
 (segment (start 158 49.5) (end 172.75 49.5) (width 0.25) (layer F.Cu) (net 14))
 (segment (start 157.42 50.08) (end 158 49.5) (width 0.25) (layer F.Cu) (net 14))
 (segment (start 194.49 48) (end 194.75 47.74) (width 0.25) (layer F.Cu) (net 14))
 (segment (start 159.96 52.25) (end 159.96 51.04) (width 0.25) (layer F.Cu) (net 15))
 (segment (start 192.97 50.28) (end 194.75 50.28) (width 0.25) (layer F.Cu) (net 15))
 (segment (start 192.5 50.75) (end 192.97 50.28) (width 0.25) (layer F.Cu) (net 15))
 (segment (start 192.5 53) (end 192.5 50.75) (width 0.25) (layer F.Cu) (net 15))
 (segment (start 191.5 54) (end 192.5 53) (width 0.25) (layer F.Cu) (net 15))
 (segment (start 172 54) (end 191.5 54) (width 0.25) (layer F.Cu) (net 15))
 (segment (start 171.5 53.5) (end 172 54) (width 0.25) (layer F.Cu) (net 15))
 (segment (start 171.5 50.75) (end 171.5 53.5) (width 0.25) (layer F.Cu) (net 15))
 (segment (start 171.25 50.5) (end 171.5 50.75) (width 0.25) (layer F.Cu) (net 15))
 (segment (start 160.5 50.5) (end 171.25 50.5) (width 0.25) (layer F.Cu) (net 15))
 (segment (start 159.96 51.04) (end 160.5 50.5) (width 0.25) (layer F.Cu) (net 15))
 (segment (start 193.5 57.75) (end 195.25 57.75) (width 0.25) (layer F.Cu) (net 16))
 (segment (start 154.88 55.63) (end 155.75 56.5) (width 0.25) (layer F.Cu) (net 16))
 (segment (start 155.75 56.5) (end 192.25 56.5) (width 0.25) (layer F.Cu) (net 16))
 (segment (start 192.25 56.5) (end 193.5 57.75) (width 0.25) (layer F.Cu) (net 16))
 (segment (start 154.88 52.25) (end 154.88 55.63) (width 0.25) (layer F.Cu) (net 16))
 (segment (start 195.93 52.82) (end 196.5 53.39) (width 0.25) (layer F.Cu) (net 16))
 (segment (start 196.5 53.39) (end 196.5 56.5) (width 0.25) (layer F.Cu) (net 16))
 (segment (start 196.5 56.5) (end 195.25 57.75) (width 0.25) (layer F.Cu) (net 16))
 (segment (start 195.93 52.82) (end 194.75 52.82) (width 0.25) (layer F.Cu) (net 16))
 (segment (start 162.5 52.25) (end 162.5 54.5) (width 0.25) (layer F.Cu) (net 17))
 (segment (start 163.25 55.25) (end 194.64 55.25) (width 0.25) (layer F.Cu) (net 17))
 (segment (start 162.5 54.5) (end 163.25 55.25) (width 0.25) (layer F.Cu) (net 17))
 (segment (start 194.64 55.25) (end 194.75 55.36) (width 0.25) (layer F.Cu) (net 17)))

